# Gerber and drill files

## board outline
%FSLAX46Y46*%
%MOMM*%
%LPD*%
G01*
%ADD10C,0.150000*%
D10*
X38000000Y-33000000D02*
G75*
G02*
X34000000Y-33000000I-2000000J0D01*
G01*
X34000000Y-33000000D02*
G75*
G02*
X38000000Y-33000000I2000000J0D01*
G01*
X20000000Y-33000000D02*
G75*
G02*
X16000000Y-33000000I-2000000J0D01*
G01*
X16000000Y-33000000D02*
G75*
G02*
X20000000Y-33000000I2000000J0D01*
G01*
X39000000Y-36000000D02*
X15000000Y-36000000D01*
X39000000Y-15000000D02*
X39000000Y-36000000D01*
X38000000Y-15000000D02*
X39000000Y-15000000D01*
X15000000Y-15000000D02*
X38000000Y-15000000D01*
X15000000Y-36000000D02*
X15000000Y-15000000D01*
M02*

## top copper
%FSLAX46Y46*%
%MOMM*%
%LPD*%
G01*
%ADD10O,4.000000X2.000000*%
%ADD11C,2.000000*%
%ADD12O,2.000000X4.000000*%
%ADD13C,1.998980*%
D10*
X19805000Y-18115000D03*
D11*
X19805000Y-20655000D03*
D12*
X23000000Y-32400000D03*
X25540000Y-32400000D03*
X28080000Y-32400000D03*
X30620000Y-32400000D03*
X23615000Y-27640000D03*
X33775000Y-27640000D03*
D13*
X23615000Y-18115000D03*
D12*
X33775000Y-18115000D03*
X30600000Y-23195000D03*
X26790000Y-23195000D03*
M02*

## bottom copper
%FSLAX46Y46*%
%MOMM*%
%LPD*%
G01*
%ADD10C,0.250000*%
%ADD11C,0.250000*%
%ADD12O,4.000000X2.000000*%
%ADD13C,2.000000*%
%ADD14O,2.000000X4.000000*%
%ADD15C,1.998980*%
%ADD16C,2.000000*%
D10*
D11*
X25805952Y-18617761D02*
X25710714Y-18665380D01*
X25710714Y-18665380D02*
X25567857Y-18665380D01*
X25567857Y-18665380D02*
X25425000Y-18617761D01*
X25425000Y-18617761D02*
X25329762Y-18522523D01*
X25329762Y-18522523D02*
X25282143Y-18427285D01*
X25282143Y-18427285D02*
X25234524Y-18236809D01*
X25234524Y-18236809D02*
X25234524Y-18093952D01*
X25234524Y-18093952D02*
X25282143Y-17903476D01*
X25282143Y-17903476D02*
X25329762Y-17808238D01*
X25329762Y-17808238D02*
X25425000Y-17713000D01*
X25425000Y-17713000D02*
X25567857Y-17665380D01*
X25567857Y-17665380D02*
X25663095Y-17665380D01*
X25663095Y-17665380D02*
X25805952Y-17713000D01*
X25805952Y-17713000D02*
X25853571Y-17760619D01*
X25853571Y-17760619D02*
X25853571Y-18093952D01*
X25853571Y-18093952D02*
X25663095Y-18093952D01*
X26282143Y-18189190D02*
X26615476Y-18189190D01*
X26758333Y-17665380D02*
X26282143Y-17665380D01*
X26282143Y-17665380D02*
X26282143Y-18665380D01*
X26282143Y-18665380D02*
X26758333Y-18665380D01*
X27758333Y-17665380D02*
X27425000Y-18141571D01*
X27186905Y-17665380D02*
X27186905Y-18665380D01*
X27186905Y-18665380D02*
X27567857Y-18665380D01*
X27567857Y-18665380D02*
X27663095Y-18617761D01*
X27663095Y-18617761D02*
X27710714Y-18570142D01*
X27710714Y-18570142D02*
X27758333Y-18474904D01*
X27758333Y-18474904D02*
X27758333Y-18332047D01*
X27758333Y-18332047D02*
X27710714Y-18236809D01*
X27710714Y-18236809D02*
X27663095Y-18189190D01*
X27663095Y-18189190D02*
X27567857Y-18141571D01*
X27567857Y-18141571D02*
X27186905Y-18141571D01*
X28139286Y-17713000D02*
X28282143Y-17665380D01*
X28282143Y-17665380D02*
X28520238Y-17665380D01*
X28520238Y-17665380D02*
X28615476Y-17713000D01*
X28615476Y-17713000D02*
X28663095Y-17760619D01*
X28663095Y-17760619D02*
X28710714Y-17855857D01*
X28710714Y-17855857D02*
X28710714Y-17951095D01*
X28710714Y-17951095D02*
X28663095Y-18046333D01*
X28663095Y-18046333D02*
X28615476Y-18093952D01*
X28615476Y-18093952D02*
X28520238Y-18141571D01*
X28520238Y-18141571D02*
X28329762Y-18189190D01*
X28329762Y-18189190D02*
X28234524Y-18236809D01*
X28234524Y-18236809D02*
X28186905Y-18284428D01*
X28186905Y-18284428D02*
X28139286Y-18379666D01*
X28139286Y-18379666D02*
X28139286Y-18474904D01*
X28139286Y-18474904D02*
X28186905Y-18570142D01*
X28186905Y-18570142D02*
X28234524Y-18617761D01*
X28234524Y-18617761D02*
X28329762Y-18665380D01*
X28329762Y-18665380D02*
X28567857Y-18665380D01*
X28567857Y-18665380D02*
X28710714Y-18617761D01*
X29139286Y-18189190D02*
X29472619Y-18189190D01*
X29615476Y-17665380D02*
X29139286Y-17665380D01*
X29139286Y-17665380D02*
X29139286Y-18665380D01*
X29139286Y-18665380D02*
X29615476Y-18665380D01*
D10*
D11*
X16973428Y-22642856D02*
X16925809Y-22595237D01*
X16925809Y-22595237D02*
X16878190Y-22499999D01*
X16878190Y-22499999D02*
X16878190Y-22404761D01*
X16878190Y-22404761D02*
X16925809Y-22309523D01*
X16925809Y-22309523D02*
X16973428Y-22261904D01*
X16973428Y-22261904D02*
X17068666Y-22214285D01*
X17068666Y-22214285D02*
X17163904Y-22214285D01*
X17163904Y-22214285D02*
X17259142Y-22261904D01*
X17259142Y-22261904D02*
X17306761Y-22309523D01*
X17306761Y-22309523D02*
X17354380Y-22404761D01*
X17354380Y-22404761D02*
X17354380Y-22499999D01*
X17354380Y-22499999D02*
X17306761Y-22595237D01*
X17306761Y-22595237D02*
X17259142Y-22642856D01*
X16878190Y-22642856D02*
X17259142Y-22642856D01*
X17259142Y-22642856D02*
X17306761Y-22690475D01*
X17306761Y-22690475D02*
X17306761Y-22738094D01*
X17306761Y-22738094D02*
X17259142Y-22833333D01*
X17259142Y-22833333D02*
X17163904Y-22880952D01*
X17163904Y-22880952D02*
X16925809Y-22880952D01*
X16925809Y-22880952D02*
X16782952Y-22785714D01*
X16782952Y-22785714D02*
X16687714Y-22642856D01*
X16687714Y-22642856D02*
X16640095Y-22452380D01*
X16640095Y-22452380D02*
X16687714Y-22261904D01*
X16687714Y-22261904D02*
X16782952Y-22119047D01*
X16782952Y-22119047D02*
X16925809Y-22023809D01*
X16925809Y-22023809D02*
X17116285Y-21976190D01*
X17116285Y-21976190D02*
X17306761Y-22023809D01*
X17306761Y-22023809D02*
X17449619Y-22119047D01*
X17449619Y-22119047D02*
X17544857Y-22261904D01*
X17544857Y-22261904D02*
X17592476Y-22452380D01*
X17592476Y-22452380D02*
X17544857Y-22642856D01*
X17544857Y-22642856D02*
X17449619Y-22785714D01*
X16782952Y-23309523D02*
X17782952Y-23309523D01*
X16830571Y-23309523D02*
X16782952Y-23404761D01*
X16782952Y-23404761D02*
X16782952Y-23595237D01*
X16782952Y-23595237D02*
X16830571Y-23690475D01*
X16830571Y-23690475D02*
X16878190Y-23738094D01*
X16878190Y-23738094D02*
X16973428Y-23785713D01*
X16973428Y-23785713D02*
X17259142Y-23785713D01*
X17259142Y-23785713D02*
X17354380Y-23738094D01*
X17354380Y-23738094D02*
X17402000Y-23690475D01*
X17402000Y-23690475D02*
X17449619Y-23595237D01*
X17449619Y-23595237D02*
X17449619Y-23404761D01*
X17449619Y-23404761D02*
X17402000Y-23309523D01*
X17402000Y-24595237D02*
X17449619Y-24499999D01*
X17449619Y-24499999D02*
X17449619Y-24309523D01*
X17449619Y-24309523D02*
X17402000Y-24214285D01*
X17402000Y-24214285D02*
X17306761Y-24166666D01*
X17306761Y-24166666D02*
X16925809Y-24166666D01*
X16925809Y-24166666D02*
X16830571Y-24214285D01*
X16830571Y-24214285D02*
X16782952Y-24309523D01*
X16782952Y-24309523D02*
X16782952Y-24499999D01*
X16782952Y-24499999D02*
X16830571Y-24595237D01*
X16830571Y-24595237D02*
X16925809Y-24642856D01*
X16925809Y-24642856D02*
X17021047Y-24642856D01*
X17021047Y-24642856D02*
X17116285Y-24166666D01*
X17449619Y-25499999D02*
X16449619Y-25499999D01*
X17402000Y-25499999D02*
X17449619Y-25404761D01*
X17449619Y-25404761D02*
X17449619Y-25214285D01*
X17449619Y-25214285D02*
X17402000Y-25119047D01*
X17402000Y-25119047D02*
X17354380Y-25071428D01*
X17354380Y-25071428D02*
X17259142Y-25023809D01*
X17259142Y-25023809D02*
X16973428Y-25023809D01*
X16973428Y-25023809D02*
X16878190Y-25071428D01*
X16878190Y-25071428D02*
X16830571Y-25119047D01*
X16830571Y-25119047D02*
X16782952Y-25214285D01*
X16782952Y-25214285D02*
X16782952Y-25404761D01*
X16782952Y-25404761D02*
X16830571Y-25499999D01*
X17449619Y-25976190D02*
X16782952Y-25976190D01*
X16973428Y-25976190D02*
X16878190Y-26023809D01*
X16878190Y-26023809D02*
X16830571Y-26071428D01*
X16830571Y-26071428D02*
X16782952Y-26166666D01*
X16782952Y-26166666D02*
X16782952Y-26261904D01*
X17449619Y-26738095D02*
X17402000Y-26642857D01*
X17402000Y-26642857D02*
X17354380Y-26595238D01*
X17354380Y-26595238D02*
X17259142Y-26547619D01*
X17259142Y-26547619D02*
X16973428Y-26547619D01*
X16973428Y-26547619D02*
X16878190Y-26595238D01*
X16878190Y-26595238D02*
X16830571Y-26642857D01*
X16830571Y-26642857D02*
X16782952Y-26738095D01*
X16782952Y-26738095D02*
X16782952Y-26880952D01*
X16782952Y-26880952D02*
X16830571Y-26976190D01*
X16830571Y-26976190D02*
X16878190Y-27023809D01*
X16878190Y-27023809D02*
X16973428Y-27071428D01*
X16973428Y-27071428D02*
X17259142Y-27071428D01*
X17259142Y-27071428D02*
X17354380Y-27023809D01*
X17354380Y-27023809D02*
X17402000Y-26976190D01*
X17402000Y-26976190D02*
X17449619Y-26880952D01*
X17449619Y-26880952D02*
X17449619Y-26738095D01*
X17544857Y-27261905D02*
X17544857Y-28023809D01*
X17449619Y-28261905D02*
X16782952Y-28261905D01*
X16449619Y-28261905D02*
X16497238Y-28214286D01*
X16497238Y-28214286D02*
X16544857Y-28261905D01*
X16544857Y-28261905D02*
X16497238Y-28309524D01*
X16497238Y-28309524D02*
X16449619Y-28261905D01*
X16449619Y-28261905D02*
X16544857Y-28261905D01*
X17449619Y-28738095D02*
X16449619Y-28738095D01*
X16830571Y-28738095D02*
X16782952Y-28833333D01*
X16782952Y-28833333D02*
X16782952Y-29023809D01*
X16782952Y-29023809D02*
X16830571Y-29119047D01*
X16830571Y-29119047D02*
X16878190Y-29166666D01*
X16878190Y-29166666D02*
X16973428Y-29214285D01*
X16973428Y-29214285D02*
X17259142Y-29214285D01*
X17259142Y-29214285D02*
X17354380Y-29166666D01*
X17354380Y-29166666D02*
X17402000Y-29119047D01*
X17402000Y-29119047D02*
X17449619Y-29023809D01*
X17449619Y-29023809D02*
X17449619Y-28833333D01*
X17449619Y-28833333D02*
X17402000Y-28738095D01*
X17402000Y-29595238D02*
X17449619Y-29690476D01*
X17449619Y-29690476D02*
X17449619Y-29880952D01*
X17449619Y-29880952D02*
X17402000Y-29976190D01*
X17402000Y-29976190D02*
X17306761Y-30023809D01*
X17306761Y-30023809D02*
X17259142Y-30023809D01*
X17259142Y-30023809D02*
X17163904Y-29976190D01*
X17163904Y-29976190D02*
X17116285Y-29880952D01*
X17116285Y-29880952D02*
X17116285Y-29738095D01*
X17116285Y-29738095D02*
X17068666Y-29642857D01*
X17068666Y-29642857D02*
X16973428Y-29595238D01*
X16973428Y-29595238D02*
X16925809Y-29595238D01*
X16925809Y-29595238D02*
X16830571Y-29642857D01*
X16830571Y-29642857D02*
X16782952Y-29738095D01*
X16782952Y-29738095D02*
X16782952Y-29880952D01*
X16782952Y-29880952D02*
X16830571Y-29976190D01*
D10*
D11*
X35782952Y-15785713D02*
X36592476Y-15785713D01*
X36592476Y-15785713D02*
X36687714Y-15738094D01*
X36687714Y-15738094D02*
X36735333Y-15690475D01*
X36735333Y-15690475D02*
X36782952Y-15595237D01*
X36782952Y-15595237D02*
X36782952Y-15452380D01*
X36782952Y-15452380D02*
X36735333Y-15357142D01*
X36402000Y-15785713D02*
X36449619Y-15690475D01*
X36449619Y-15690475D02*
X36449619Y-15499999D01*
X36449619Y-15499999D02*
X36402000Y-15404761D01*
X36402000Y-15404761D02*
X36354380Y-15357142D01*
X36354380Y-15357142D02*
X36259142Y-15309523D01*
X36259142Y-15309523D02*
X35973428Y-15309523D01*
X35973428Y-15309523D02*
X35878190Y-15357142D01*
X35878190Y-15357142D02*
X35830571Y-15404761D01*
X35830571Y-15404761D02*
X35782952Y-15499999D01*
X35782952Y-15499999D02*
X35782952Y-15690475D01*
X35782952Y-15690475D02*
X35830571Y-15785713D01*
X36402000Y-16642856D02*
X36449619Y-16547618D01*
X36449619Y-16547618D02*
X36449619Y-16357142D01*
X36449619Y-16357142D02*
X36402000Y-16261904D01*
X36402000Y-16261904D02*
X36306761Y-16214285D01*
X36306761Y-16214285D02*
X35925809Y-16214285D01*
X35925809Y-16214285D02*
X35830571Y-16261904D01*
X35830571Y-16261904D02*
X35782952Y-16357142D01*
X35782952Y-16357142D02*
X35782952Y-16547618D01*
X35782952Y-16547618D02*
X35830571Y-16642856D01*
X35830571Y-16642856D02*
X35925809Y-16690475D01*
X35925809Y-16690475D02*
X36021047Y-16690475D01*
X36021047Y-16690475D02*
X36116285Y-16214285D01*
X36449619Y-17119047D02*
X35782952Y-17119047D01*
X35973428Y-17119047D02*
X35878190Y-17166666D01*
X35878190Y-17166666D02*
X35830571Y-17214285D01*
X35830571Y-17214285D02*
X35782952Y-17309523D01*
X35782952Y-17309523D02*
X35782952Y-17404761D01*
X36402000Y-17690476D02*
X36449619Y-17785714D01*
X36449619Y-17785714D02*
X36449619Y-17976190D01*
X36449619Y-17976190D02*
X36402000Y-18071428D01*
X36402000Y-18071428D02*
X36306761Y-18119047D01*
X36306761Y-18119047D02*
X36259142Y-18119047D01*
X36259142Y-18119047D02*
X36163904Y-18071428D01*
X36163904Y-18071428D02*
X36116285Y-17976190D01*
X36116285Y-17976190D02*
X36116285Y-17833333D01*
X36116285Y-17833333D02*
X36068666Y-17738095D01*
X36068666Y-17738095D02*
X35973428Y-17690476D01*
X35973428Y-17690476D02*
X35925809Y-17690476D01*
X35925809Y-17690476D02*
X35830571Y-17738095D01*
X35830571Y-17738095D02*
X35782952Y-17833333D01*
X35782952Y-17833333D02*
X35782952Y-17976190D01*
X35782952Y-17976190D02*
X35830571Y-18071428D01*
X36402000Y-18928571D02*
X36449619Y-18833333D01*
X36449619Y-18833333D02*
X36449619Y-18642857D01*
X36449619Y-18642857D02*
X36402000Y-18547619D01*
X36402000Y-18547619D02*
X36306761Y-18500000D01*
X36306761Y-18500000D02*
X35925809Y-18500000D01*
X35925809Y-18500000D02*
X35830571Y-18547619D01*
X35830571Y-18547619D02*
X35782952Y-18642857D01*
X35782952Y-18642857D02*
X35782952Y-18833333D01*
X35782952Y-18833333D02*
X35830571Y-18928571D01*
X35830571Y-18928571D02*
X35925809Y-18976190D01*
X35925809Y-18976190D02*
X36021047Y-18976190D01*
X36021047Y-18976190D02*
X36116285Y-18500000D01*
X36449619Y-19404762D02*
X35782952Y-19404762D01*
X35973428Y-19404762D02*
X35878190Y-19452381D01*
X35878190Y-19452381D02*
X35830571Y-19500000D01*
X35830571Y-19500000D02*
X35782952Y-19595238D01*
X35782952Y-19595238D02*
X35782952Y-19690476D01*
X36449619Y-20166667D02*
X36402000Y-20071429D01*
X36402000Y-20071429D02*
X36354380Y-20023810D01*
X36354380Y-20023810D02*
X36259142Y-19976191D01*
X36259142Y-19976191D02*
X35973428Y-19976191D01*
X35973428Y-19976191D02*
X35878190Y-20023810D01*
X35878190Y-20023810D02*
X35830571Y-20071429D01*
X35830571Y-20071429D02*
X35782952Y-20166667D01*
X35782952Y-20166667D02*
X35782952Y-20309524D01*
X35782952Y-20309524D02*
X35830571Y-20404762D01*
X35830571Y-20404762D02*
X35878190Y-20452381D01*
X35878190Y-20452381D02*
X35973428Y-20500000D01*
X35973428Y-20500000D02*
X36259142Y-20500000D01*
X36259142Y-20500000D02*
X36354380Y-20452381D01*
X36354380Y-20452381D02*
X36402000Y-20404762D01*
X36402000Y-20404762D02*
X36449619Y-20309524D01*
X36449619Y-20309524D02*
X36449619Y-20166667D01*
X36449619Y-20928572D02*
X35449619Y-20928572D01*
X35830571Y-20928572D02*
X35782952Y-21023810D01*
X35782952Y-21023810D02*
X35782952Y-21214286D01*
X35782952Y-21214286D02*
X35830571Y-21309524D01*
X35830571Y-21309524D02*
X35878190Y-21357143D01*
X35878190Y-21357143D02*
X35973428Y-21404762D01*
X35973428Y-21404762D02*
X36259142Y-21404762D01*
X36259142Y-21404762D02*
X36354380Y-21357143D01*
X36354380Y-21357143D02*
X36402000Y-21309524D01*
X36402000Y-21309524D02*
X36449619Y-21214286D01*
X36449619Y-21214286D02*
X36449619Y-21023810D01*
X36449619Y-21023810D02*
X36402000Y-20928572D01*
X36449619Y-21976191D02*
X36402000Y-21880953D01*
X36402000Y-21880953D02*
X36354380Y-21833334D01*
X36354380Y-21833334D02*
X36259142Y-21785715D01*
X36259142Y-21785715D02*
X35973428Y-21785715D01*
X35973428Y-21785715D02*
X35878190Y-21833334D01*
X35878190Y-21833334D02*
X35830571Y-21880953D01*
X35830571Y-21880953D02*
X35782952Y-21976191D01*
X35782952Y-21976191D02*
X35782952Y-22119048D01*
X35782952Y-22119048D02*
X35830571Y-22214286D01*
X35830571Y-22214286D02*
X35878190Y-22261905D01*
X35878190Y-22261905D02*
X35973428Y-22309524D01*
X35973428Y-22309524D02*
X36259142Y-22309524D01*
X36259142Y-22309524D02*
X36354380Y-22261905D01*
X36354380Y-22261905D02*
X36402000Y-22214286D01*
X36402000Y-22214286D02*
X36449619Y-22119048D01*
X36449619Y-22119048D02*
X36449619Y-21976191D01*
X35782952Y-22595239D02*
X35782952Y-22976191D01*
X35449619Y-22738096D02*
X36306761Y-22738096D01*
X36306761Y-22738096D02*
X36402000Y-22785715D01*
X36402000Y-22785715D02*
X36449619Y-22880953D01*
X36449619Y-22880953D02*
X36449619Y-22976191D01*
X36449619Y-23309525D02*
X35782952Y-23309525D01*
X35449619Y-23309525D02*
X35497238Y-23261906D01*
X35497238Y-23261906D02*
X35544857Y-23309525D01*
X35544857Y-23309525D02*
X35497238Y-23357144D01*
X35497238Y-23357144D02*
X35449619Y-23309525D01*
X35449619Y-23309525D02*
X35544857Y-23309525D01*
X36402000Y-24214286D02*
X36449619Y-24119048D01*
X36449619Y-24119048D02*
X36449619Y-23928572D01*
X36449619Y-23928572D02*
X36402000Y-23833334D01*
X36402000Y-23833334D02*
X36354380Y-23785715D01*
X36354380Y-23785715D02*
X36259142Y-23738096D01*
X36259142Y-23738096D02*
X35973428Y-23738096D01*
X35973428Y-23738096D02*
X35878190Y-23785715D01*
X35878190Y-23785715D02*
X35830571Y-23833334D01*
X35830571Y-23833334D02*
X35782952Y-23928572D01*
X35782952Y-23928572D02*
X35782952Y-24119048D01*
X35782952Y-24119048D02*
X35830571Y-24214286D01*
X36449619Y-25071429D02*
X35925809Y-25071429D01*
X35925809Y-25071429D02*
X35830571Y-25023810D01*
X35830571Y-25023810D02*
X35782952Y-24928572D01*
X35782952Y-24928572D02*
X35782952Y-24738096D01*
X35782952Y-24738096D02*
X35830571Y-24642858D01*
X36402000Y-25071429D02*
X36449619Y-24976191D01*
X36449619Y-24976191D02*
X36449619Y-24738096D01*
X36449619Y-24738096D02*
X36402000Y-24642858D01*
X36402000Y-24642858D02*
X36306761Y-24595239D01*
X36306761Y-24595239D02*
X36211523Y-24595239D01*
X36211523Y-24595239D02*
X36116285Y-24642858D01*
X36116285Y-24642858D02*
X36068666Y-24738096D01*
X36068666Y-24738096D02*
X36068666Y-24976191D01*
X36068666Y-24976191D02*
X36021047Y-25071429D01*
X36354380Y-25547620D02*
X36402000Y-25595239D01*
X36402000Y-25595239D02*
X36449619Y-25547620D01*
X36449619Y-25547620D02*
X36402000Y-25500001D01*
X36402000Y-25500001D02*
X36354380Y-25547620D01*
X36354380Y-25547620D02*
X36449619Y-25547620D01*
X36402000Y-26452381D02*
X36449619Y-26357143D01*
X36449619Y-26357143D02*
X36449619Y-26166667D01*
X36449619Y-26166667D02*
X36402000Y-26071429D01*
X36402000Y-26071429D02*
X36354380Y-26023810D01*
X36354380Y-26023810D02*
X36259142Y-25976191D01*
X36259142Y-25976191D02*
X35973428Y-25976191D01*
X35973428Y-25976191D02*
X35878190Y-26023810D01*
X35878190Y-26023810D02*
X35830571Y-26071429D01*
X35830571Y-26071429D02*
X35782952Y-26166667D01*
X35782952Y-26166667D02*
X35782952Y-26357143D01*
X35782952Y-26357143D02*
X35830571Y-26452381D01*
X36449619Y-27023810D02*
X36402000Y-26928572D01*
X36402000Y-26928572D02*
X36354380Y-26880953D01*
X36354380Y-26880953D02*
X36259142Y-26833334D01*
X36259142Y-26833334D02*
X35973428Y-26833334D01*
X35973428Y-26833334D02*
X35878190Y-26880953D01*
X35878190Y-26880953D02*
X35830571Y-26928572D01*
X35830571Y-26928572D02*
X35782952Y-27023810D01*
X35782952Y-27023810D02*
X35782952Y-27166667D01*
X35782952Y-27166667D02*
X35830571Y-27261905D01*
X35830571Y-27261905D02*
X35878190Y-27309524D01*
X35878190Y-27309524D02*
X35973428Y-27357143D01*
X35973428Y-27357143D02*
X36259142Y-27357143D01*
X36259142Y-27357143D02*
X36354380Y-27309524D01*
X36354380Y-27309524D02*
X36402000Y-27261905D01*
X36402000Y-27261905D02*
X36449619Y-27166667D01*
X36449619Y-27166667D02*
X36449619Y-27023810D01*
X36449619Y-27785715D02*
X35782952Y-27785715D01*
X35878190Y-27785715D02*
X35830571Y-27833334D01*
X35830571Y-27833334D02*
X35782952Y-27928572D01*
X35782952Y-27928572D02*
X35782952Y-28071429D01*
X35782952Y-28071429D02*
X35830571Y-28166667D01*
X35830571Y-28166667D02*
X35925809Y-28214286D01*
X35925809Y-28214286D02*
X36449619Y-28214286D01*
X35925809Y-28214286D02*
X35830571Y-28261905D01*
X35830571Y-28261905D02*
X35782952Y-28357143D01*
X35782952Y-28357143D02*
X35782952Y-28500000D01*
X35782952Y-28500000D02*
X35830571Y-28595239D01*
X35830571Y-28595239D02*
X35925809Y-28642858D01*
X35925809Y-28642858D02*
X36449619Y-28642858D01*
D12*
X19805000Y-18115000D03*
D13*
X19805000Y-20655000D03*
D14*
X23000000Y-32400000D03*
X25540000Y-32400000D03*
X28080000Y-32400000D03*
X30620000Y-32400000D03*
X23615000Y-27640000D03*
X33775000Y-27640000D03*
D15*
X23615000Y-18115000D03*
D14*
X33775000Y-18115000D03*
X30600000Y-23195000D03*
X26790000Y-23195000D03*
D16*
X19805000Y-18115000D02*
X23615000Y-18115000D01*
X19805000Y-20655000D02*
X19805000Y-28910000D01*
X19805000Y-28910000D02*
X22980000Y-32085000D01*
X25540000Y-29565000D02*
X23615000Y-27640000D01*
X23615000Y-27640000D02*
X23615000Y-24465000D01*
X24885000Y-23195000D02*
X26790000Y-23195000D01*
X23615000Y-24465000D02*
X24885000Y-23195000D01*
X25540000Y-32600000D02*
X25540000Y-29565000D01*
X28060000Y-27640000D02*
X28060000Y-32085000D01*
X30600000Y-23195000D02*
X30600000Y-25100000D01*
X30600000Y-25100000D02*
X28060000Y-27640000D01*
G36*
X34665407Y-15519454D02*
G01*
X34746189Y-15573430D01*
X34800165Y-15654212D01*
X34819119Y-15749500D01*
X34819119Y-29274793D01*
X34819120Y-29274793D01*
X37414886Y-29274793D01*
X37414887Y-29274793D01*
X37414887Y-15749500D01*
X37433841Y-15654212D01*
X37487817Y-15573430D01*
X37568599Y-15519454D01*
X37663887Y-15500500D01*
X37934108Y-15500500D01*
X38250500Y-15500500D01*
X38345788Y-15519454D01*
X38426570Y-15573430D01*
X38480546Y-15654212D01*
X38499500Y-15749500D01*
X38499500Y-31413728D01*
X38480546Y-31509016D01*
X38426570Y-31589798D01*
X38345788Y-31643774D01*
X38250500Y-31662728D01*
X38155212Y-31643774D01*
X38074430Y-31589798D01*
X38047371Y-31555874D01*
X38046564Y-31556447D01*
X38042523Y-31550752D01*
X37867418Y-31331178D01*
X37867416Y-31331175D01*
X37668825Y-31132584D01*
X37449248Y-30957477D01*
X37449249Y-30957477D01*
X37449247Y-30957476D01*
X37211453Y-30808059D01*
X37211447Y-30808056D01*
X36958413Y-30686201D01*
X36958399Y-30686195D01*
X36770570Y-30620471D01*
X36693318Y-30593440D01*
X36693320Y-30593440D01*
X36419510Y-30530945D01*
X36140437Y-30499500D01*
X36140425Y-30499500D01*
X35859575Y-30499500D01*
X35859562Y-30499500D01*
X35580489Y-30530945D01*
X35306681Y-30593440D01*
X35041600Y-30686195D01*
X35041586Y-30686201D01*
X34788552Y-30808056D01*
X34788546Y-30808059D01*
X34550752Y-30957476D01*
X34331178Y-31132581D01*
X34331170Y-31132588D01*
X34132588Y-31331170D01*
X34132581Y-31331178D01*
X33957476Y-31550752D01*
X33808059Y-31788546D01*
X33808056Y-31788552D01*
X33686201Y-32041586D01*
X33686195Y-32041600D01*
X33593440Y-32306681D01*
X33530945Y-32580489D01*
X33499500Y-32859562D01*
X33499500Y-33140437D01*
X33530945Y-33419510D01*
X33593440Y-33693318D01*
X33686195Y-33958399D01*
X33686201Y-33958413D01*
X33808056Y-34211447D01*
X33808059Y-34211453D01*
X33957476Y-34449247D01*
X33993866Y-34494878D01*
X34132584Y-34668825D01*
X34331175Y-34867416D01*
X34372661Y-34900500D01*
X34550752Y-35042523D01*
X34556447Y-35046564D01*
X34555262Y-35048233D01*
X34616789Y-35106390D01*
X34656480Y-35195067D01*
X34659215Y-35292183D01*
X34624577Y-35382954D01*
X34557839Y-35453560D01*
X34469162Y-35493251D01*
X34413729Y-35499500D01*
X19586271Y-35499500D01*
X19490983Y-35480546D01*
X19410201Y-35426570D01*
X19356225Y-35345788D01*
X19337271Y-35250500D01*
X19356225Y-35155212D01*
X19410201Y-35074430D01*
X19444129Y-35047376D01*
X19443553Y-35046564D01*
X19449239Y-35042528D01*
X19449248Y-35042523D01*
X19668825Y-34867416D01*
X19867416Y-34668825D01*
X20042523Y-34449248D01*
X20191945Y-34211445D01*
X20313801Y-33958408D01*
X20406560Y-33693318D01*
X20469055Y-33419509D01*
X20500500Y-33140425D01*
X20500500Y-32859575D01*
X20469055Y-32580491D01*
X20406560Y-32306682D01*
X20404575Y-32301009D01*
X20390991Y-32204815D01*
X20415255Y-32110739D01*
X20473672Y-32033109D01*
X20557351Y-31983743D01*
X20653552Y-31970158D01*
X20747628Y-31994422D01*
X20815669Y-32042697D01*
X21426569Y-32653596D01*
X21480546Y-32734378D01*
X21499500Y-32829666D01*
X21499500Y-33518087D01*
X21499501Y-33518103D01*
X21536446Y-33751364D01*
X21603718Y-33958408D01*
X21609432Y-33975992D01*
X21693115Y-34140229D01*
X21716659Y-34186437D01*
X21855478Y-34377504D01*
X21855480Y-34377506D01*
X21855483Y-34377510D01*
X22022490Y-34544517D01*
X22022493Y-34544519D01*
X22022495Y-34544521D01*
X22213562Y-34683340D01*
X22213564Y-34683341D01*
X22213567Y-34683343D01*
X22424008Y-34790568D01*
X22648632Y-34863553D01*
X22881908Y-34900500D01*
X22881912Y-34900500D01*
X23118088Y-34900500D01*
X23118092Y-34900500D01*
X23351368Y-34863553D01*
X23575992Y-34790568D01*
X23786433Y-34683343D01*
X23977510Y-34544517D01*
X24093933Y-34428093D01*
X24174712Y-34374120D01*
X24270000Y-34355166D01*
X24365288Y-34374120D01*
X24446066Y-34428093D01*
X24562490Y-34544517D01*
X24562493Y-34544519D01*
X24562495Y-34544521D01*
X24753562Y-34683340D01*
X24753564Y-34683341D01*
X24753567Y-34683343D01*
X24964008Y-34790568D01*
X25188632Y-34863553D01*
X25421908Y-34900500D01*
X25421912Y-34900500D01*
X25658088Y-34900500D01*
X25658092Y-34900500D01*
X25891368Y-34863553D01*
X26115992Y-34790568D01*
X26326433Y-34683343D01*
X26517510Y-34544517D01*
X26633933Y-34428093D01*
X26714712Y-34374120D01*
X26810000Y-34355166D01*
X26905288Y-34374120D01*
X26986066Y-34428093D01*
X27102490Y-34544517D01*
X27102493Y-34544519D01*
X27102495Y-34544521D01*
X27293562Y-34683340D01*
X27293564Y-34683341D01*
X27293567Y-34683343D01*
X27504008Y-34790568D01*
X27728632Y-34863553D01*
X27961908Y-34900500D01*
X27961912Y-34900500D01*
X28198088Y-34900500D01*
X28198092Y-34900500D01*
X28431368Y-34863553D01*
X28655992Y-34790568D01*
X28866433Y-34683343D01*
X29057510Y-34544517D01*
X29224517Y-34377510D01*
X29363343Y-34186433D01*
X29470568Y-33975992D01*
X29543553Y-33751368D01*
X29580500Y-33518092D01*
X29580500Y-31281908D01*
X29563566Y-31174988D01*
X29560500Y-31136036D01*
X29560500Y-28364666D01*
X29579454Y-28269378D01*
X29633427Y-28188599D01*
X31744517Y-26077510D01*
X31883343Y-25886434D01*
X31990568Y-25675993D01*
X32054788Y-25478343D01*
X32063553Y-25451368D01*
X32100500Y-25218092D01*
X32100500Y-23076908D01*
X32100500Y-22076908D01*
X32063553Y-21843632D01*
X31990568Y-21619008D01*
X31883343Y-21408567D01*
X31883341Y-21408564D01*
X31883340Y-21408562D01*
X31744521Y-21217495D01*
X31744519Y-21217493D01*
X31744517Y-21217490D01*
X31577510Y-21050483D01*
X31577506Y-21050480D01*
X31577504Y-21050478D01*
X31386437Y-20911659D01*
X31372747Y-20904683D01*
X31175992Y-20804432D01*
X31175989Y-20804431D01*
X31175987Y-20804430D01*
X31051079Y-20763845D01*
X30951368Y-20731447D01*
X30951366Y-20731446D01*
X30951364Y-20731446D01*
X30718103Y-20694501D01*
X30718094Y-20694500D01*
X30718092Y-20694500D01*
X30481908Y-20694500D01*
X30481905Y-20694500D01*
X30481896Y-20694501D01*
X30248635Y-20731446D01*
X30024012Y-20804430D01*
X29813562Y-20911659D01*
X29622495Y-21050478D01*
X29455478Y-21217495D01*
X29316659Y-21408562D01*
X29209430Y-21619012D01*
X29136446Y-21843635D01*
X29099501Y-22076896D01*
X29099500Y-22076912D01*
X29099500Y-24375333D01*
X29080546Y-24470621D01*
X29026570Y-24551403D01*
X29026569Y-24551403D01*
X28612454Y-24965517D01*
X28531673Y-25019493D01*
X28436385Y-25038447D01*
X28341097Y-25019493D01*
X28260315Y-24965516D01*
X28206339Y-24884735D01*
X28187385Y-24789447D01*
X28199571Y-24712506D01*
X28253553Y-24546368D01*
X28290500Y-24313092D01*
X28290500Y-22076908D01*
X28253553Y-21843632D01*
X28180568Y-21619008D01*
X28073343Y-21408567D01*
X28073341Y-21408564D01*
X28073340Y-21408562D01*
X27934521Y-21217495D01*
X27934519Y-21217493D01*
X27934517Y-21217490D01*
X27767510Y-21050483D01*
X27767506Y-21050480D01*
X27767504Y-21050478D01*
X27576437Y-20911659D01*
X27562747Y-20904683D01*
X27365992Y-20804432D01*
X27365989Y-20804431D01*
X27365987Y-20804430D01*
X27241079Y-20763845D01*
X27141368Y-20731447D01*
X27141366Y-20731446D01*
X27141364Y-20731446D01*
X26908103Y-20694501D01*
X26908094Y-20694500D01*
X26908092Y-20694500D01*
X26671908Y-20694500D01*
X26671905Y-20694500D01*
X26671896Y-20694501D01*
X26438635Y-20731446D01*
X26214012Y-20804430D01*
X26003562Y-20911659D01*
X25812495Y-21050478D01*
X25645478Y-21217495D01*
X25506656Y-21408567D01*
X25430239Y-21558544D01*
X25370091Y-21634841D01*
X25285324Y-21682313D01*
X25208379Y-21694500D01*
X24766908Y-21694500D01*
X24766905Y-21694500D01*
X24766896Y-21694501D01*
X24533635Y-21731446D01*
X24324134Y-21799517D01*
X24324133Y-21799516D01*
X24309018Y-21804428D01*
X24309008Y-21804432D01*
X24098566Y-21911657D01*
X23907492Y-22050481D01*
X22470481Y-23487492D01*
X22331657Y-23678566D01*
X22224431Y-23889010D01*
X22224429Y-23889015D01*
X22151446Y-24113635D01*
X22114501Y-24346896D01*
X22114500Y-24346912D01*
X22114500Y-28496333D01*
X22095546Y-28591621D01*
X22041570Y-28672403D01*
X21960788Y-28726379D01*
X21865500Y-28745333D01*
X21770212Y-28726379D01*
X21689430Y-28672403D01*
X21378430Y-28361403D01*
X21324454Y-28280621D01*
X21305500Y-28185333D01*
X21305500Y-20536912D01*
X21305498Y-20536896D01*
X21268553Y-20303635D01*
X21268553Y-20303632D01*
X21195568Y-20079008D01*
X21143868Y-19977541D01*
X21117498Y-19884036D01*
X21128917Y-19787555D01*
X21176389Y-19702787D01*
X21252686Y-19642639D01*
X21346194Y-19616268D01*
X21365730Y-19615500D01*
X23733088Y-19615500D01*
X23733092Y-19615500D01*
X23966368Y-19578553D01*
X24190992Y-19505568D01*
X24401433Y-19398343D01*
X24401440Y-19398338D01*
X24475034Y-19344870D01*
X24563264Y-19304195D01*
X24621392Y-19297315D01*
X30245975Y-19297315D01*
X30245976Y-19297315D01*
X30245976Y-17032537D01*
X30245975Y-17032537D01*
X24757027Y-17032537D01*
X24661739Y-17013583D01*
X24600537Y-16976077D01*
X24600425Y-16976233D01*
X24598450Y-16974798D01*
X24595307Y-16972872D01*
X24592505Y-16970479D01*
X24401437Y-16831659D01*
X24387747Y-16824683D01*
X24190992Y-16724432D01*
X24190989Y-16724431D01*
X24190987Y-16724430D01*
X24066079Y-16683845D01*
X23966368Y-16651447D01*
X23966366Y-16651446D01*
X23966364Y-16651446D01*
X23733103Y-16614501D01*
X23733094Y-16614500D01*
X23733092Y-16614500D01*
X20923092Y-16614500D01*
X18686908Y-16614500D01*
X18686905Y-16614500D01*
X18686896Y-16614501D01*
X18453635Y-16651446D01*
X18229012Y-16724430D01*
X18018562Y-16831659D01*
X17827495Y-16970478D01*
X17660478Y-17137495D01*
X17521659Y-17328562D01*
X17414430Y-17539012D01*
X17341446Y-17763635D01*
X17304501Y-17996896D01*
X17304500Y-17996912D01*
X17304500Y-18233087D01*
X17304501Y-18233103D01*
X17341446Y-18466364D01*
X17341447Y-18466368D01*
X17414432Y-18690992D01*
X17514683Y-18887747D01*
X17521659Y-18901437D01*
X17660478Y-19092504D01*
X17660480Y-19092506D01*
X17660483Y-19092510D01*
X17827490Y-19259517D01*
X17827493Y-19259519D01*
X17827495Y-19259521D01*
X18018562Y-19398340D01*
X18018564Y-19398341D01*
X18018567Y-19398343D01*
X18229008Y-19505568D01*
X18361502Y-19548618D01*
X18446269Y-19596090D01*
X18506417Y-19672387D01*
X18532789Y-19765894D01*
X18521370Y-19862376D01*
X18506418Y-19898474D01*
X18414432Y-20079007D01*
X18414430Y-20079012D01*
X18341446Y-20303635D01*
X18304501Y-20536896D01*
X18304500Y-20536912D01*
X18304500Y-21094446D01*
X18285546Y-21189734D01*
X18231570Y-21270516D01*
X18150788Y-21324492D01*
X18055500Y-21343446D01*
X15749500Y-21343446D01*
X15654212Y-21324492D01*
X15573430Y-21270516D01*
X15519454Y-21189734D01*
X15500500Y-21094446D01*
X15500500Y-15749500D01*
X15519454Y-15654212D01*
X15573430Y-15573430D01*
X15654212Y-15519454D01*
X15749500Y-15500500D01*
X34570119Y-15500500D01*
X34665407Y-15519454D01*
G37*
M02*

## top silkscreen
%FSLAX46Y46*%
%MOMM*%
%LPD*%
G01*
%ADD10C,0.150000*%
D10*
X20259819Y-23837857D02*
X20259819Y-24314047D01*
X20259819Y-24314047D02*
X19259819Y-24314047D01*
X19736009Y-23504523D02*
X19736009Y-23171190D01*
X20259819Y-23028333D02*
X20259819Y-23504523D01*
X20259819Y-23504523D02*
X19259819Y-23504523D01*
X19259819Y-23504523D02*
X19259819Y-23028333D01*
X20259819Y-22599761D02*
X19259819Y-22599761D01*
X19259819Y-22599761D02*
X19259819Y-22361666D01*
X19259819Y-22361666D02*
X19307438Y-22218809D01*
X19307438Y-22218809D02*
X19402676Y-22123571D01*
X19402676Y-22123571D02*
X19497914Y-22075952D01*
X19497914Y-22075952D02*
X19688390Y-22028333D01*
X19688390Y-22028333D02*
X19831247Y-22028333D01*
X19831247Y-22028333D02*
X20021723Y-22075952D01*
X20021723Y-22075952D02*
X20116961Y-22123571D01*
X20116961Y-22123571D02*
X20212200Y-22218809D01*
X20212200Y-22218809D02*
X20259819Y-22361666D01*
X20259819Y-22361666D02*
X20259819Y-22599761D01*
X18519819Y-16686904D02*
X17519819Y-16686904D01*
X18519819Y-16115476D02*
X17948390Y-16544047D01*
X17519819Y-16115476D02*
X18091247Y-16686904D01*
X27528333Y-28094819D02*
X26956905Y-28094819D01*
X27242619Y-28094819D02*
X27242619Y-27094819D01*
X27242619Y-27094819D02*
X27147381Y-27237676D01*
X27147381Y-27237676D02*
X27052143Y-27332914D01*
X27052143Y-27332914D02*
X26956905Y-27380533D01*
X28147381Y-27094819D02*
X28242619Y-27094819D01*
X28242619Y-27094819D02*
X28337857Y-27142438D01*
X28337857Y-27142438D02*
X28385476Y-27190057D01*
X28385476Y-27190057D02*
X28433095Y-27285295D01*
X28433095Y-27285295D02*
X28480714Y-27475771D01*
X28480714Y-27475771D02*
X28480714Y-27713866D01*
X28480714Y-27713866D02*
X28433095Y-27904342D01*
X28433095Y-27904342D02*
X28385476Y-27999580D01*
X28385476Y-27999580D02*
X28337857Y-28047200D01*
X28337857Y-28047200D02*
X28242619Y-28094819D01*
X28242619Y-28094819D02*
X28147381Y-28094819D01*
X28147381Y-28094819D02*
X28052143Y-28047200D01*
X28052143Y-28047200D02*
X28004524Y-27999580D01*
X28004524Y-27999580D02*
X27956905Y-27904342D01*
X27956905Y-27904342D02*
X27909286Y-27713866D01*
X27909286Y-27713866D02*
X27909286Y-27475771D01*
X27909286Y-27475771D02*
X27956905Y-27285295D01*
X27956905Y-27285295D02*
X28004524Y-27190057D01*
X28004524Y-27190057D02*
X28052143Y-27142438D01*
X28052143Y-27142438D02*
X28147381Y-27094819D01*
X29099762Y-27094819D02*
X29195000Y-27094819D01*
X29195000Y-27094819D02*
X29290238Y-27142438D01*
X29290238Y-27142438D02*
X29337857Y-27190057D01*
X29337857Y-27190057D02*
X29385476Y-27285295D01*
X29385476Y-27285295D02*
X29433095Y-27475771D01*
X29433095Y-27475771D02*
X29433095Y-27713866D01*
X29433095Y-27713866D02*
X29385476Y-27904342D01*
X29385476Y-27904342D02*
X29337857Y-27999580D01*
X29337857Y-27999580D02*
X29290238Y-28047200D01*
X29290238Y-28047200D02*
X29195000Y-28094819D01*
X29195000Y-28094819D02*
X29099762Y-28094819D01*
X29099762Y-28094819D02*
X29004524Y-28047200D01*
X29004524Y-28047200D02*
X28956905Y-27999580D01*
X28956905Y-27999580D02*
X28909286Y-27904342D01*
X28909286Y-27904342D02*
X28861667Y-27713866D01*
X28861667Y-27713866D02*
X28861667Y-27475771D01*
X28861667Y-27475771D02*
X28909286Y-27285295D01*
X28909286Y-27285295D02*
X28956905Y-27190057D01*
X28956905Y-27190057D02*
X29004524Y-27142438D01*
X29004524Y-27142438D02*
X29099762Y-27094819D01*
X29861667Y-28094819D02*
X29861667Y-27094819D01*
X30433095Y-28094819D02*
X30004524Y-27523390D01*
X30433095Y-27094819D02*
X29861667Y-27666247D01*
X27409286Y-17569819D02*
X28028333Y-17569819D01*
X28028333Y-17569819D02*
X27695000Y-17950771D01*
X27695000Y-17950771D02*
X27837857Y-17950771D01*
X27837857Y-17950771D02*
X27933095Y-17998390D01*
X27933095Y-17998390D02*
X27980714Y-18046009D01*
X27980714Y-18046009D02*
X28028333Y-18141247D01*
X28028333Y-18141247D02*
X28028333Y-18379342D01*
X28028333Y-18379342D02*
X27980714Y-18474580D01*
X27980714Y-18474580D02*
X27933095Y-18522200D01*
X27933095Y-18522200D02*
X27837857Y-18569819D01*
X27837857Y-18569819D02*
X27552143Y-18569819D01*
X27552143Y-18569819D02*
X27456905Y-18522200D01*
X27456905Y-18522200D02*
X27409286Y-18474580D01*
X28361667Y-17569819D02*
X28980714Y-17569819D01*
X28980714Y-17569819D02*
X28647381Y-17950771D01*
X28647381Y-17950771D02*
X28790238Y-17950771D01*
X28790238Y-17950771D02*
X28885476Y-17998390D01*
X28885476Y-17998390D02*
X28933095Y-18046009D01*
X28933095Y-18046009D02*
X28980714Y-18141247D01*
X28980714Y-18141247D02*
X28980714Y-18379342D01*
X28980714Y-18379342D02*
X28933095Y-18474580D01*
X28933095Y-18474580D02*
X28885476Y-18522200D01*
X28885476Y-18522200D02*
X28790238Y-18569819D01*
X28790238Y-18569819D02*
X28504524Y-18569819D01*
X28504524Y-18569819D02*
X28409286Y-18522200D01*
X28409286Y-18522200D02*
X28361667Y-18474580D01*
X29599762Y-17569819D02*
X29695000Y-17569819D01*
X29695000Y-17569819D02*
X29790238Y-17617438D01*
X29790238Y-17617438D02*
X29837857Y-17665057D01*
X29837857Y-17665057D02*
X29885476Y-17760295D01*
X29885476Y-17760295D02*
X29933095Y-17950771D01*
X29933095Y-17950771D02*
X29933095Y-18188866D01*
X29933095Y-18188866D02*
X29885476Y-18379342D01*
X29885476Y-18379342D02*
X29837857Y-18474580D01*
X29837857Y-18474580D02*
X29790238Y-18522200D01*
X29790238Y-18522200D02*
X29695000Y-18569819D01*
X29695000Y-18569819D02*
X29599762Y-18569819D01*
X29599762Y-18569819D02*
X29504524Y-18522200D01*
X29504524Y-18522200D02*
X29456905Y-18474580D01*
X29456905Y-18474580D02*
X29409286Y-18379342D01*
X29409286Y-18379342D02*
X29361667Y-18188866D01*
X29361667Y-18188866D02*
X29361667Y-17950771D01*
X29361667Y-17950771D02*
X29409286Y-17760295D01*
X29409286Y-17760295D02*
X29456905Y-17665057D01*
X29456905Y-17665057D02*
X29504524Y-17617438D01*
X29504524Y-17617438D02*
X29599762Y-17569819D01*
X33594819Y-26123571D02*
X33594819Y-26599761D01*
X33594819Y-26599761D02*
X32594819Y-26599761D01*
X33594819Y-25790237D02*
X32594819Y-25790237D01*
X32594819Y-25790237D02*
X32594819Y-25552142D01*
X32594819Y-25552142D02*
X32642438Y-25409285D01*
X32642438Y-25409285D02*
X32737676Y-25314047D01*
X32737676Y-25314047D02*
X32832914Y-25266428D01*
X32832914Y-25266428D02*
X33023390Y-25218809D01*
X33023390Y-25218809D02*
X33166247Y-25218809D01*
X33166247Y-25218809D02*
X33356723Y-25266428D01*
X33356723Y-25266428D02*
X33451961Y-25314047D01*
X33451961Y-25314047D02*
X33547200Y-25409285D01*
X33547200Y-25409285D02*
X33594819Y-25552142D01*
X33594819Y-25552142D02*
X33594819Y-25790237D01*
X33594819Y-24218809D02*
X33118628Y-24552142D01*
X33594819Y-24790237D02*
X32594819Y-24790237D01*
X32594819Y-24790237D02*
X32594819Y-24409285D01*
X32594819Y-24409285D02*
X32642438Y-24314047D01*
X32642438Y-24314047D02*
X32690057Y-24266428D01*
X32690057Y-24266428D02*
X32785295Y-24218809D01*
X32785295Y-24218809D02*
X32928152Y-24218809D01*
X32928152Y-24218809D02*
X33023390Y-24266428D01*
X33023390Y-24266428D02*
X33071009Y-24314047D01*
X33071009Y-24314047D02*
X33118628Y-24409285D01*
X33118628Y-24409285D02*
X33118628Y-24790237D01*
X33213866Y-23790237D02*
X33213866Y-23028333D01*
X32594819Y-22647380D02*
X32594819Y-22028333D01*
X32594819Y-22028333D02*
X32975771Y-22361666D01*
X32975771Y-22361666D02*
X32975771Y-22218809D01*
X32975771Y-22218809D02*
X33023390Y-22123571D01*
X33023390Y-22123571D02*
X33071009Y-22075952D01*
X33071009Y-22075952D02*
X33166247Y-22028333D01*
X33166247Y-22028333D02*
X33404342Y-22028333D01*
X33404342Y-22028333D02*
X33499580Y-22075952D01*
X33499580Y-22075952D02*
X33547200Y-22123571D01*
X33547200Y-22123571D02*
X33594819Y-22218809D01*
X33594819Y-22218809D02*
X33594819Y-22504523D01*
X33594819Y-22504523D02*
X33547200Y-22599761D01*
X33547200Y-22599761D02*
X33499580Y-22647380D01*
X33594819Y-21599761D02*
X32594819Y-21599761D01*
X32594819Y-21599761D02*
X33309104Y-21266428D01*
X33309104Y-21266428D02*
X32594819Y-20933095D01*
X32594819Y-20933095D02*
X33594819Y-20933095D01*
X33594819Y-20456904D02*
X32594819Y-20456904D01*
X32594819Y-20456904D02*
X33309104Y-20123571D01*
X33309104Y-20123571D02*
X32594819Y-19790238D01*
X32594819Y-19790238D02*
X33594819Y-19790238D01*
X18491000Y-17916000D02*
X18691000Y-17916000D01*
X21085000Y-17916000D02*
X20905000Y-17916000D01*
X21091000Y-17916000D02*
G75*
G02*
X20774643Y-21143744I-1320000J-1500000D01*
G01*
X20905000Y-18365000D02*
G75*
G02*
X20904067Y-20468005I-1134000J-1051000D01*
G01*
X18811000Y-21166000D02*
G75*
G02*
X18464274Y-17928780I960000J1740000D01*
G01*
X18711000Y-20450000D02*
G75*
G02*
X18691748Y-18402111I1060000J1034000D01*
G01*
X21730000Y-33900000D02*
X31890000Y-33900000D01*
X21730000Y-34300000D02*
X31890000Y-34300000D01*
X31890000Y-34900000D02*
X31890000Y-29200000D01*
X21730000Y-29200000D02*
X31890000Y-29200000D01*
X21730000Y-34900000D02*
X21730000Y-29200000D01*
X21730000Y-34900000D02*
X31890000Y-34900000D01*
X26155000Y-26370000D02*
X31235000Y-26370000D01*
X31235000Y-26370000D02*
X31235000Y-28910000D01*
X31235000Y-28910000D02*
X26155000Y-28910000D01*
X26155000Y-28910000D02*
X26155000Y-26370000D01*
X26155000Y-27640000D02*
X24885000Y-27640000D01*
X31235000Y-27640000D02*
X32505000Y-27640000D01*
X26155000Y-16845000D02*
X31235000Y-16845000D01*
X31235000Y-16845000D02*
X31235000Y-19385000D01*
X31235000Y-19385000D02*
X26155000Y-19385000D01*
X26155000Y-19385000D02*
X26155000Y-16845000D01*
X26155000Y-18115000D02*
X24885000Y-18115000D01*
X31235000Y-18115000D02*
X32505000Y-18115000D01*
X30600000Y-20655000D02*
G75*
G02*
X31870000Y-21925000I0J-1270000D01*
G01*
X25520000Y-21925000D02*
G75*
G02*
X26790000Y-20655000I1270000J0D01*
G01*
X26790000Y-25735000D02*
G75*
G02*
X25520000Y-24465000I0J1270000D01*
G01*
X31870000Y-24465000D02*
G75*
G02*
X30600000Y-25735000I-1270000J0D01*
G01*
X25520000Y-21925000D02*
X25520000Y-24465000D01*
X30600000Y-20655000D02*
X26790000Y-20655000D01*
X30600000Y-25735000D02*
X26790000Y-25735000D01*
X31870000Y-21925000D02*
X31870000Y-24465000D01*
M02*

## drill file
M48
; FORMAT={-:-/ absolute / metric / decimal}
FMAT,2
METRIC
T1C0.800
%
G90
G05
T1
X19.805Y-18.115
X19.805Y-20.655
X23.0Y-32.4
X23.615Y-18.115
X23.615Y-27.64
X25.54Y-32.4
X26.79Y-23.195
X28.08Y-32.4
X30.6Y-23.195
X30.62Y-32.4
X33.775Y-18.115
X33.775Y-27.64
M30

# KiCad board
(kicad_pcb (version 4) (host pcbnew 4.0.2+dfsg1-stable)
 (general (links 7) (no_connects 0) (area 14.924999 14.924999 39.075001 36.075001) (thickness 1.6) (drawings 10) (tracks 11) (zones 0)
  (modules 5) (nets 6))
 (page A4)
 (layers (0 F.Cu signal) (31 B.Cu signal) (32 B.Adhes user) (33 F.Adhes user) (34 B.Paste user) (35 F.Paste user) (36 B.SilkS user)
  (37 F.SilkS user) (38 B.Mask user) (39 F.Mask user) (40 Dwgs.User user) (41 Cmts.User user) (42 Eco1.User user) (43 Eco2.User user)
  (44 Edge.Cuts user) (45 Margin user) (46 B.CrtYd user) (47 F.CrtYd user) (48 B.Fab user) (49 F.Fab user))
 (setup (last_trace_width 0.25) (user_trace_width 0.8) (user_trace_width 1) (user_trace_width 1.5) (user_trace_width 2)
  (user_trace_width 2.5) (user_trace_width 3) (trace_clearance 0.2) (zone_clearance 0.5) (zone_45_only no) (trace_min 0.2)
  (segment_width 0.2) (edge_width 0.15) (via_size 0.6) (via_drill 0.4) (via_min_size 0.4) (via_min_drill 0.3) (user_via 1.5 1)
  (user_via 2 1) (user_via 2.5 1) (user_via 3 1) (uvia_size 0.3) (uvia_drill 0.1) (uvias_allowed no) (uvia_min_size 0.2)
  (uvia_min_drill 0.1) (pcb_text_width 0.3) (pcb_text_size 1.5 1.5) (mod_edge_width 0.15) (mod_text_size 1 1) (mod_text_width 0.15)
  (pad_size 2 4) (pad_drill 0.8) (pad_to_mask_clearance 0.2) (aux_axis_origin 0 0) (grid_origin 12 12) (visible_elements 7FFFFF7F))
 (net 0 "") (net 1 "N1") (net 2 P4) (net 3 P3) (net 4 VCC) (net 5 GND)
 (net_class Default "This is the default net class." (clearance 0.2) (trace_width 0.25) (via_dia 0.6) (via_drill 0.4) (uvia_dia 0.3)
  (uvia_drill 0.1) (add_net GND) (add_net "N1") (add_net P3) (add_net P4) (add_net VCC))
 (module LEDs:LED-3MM (layer F.Cu) (at 19.805 18.115 270)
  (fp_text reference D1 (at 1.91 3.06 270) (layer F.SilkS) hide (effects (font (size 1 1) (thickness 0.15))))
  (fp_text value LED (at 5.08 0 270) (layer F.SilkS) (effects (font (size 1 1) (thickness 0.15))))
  (fp_line (start -0.199 1.314) (end -0.199 1.114) (layer F.SilkS) (width 0.15))
  (fp_line (start -0.199 -1.28) (end -0.199 -1.1) (layer F.SilkS) (width 0.15))
  (fp_arc (start 1.301 0.034) (end -0.199 -1.286) (angle 108.5) (layer F.SilkS) (width 0.15))
  (fp_arc (start 1.301 0.034) (end 0.25 -1.1) (angle 85.7) (layer F.SilkS) (width 0.15))
  (fp_arc (start 1.311 0.034) (end 3.051 0.994) (angle 110) (layer F.SilkS) (width 0.15))
  (fp_arc (start 1.301 0.034) (end 2.335 1.094) (angle 87.5) (layer F.SilkS) (width 0.15))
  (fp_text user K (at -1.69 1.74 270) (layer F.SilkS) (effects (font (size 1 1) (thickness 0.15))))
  (pad 1 thru_hole oval (at 0 0) (size 4 2) (drill 0.8) (layers *.Cu) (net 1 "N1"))
  (pad 2 thru_hole circle (at 2.54 0 270) (size 2 2) (drill 0.8) (layers *.Cu) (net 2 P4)))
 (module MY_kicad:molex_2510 (layer F.Cu) (at 23 32.4)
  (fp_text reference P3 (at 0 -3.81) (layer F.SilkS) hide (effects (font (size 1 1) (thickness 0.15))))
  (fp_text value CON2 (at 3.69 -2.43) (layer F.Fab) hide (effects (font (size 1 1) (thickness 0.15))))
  (fp_line (start -1.27 1.5) (end 8.89 1.5) (layer F.SilkS) (width 0.15))
  (fp_line (start -1.27 1.9) (end 8.89 1.9) (layer F.SilkS) (width 0.15))
  (fp_line (start 8.89 2.5) (end 8.89 -3.2) (layer F.SilkS) (width 0.15))
  (fp_line (start -1.27 -3.2) (end 8.89 -3.2) (layer F.SilkS) (width 0.15))
  (fp_line (start -1.27 2.5) (end -1.27 -3.2) (layer F.SilkS) (width 0.15))
  (fp_line (start -1.27 2.5) (end 8.89 2.5) (layer F.SilkS) (width 0.15))
  (pad 1 thru_hole oval (at 0 0) (size 2 4) (drill 0.8) (layers *.Cu) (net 2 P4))
  (pad 2 thru_hole oval (at 2.54 0) (size 2 4) (drill 0.8) (layers *.Cu) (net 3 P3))
  (pad 3 thru_hole oval (at 5.08 0) (size 2 4) (drill 0.8) (layers *.Cu) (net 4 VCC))
  (pad 4 thru_hole oval (at 7.62 0) (size 2 4) (drill 0.8) (layers *.Cu) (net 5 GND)))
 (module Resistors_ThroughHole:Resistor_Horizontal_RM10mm (layer F.Cu) (at 23.615 27.64)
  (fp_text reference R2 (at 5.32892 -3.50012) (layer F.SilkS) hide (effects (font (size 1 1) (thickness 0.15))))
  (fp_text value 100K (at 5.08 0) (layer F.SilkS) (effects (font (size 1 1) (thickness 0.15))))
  (fp_line (start 2.54 -1.27) (end 7.62 -1.27) (layer F.SilkS) (width 0.15))
  (fp_line (start 7.62 -1.27) (end 7.62 1.27) (layer F.SilkS) (width 0.15))
  (fp_line (start 7.62 1.27) (end 2.54 1.27) (layer F.SilkS) (width 0.15))
  (fp_line (start 2.54 1.27) (end 2.54 -1.27) (layer F.SilkS) (width 0.15))
  (fp_line (start 2.54 0) (end 1.27 0) (layer F.SilkS) (width 0.15))
  (fp_line (start 7.62 0) (end 8.89 0) (layer F.SilkS) (width 0.15))
  (pad 1 thru_hole oval (at 0 0) (size 2 4) (drill 0.8) (layers *.Cu) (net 3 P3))
  (pad 2 thru_hole oval (at 10.16 0) (size 2 4) (drill 0.8) (layers *.Cu) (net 5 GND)))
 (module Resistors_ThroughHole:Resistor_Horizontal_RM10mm (layer F.Cu) (at 23.615 18.115)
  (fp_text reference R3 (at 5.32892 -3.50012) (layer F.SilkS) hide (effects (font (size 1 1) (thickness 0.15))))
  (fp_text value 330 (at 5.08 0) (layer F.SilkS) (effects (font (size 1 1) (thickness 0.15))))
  (fp_line (start 2.54 -1.27) (end 7.62 -1.27) (layer F.SilkS) (width 0.15))
  (fp_line (start 7.62 -1.27) (end 7.62 1.27) (layer F.SilkS) (width 0.15))
  (fp_line (start 7.62 1.27) (end 2.54 1.27) (layer F.SilkS) (width 0.15))
  (fp_line (start 2.54 1.27) (end 2.54 -1.27) (layer F.SilkS) (width 0.15))
  (fp_line (start 2.54 0) (end 1.27 0) (layer F.SilkS) (width 0.15))
  (fp_line (start 7.62 0) (end 8.89 0) (layer F.SilkS) (width 0.15))
  (pad 1 thru_hole circle (at 0 0) (size 1.99898 1.99898) (drill 0.8) (layers *.Cu) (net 1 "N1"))
  (pad 2 thru_hole oval (at 10.16 0) (size 2 4) (drill 0.8) (layers *.Cu) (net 5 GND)))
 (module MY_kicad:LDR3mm (layer F.Cu) (at 30.6 23.195 180)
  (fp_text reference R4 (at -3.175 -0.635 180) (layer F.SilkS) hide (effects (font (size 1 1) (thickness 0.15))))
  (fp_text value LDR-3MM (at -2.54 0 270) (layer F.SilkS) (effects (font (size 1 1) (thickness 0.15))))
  (fp_arc (start 0 1.27) (end 0 2.54) (angle 90) (layer F.SilkS) (width 0.15))
  (fp_arc (start 3.81 1.27) (end 5.08 1.27) (angle 90) (layer F.SilkS) (width 0.15))
  (fp_arc (start 3.81 -1.27) (end 3.81 -2.54) (angle 90) (layer F.SilkS) (width 0.15))
  (fp_arc (start 0 -1.27) (end -1.27 -1.27) (angle 90) (layer F.SilkS) (width 0.15))
  (fp_line (start 5.08 1.27) (end 5.08 -1.27) (layer F.SilkS) (width 0.15))
  (fp_line (start 0 2.54) (end 3.81 2.54) (layer F.SilkS) (width 0.15))
  (fp_line (start 0 -2.54) (end 3.81 -2.54) (layer F.SilkS) (width 0.15))
  (fp_line (start -1.27 1.27) (end -1.27 -1.27) (layer F.SilkS) (width 0.15))
  (pad 1 thru_hole oval (at 0 0 180) (size 2 4) (drill 0.8) (layers *.Cu) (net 4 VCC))
  (pad 2 thru_hole oval (at 3.81 0 180) (size 2 4) (drill 0.8) (layers *.Cu) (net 3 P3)))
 (gr_circle (center 36 33) (end 38 33) (layer Edge.Cuts) (width 0.15))
 (gr_circle (center 18 33) (end 20 33) (layer Edge.Cuts) (width 0.15))
 (gr_line (start 39 36) (end 15 36) (angle 90) (layer Edge.Cuts) (width 0.15))
 (gr_line (start 39 15) (end 39 36) (angle 90) (layer Edge.Cuts) (width 0.15))
 (gr_line (start 38 15) (end 39 15) (angle 90) (layer Edge.Cuts) (width 0.15))
 (gr_line (start 15 15) (end 38 15) (angle 90) (layer Edge.Cuts) (width 0.15))
 (gr_line (start 15 36) (end 15 15) (angle 90) (layer Edge.Cuts) (width 0.15))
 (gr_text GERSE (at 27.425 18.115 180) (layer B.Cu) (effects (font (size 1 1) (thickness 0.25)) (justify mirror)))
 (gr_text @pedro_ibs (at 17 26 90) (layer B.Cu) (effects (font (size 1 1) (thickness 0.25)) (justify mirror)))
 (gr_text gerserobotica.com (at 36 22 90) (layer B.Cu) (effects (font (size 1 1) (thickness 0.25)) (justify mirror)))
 (segment (start 19.805 18.115) (end 23.615 18.115) (width 2) (layer B.Cu) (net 1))
 (segment (start 19.805 20.655) (end 19.805 28.91) (width 2) (layer B.Cu) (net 2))
 (segment (start 19.805 28.91) (end 22.98 32.085) (width 2) (layer B.Cu) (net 2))
 (segment (start 25.54 29.565) (end 23.615 27.64) (width 2) (layer B.Cu) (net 3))
 (segment (start 23.615 27.64) (end 23.615 24.465) (width 2) (layer B.Cu) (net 3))
 (segment (start 24.885 23.195) (end 26.79 23.195) (width 2) (layer B.Cu) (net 3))
 (segment (start 23.615 24.465) (end 24.885 23.195) (width 2) (layer B.Cu) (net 3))
 (segment (start 25.54 32.6) (end 25.54 29.565) (width 2) (layer B.Cu) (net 3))
 (segment (start 28.06 27.64) (end 28.06 32.085) (width 2) (layer B.Cu) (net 4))
 (segment (start 30.6 23.195) (end 30.6 25.1) (width 2) (layer B.Cu) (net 4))
 (segment (start 30.6 25.1) (end 28.06 27.64) (width 2) (layer B.Cu) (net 4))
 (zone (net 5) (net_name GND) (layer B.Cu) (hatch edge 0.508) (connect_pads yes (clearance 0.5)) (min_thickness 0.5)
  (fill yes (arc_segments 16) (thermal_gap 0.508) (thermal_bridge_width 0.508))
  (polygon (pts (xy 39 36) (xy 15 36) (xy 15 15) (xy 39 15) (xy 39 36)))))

